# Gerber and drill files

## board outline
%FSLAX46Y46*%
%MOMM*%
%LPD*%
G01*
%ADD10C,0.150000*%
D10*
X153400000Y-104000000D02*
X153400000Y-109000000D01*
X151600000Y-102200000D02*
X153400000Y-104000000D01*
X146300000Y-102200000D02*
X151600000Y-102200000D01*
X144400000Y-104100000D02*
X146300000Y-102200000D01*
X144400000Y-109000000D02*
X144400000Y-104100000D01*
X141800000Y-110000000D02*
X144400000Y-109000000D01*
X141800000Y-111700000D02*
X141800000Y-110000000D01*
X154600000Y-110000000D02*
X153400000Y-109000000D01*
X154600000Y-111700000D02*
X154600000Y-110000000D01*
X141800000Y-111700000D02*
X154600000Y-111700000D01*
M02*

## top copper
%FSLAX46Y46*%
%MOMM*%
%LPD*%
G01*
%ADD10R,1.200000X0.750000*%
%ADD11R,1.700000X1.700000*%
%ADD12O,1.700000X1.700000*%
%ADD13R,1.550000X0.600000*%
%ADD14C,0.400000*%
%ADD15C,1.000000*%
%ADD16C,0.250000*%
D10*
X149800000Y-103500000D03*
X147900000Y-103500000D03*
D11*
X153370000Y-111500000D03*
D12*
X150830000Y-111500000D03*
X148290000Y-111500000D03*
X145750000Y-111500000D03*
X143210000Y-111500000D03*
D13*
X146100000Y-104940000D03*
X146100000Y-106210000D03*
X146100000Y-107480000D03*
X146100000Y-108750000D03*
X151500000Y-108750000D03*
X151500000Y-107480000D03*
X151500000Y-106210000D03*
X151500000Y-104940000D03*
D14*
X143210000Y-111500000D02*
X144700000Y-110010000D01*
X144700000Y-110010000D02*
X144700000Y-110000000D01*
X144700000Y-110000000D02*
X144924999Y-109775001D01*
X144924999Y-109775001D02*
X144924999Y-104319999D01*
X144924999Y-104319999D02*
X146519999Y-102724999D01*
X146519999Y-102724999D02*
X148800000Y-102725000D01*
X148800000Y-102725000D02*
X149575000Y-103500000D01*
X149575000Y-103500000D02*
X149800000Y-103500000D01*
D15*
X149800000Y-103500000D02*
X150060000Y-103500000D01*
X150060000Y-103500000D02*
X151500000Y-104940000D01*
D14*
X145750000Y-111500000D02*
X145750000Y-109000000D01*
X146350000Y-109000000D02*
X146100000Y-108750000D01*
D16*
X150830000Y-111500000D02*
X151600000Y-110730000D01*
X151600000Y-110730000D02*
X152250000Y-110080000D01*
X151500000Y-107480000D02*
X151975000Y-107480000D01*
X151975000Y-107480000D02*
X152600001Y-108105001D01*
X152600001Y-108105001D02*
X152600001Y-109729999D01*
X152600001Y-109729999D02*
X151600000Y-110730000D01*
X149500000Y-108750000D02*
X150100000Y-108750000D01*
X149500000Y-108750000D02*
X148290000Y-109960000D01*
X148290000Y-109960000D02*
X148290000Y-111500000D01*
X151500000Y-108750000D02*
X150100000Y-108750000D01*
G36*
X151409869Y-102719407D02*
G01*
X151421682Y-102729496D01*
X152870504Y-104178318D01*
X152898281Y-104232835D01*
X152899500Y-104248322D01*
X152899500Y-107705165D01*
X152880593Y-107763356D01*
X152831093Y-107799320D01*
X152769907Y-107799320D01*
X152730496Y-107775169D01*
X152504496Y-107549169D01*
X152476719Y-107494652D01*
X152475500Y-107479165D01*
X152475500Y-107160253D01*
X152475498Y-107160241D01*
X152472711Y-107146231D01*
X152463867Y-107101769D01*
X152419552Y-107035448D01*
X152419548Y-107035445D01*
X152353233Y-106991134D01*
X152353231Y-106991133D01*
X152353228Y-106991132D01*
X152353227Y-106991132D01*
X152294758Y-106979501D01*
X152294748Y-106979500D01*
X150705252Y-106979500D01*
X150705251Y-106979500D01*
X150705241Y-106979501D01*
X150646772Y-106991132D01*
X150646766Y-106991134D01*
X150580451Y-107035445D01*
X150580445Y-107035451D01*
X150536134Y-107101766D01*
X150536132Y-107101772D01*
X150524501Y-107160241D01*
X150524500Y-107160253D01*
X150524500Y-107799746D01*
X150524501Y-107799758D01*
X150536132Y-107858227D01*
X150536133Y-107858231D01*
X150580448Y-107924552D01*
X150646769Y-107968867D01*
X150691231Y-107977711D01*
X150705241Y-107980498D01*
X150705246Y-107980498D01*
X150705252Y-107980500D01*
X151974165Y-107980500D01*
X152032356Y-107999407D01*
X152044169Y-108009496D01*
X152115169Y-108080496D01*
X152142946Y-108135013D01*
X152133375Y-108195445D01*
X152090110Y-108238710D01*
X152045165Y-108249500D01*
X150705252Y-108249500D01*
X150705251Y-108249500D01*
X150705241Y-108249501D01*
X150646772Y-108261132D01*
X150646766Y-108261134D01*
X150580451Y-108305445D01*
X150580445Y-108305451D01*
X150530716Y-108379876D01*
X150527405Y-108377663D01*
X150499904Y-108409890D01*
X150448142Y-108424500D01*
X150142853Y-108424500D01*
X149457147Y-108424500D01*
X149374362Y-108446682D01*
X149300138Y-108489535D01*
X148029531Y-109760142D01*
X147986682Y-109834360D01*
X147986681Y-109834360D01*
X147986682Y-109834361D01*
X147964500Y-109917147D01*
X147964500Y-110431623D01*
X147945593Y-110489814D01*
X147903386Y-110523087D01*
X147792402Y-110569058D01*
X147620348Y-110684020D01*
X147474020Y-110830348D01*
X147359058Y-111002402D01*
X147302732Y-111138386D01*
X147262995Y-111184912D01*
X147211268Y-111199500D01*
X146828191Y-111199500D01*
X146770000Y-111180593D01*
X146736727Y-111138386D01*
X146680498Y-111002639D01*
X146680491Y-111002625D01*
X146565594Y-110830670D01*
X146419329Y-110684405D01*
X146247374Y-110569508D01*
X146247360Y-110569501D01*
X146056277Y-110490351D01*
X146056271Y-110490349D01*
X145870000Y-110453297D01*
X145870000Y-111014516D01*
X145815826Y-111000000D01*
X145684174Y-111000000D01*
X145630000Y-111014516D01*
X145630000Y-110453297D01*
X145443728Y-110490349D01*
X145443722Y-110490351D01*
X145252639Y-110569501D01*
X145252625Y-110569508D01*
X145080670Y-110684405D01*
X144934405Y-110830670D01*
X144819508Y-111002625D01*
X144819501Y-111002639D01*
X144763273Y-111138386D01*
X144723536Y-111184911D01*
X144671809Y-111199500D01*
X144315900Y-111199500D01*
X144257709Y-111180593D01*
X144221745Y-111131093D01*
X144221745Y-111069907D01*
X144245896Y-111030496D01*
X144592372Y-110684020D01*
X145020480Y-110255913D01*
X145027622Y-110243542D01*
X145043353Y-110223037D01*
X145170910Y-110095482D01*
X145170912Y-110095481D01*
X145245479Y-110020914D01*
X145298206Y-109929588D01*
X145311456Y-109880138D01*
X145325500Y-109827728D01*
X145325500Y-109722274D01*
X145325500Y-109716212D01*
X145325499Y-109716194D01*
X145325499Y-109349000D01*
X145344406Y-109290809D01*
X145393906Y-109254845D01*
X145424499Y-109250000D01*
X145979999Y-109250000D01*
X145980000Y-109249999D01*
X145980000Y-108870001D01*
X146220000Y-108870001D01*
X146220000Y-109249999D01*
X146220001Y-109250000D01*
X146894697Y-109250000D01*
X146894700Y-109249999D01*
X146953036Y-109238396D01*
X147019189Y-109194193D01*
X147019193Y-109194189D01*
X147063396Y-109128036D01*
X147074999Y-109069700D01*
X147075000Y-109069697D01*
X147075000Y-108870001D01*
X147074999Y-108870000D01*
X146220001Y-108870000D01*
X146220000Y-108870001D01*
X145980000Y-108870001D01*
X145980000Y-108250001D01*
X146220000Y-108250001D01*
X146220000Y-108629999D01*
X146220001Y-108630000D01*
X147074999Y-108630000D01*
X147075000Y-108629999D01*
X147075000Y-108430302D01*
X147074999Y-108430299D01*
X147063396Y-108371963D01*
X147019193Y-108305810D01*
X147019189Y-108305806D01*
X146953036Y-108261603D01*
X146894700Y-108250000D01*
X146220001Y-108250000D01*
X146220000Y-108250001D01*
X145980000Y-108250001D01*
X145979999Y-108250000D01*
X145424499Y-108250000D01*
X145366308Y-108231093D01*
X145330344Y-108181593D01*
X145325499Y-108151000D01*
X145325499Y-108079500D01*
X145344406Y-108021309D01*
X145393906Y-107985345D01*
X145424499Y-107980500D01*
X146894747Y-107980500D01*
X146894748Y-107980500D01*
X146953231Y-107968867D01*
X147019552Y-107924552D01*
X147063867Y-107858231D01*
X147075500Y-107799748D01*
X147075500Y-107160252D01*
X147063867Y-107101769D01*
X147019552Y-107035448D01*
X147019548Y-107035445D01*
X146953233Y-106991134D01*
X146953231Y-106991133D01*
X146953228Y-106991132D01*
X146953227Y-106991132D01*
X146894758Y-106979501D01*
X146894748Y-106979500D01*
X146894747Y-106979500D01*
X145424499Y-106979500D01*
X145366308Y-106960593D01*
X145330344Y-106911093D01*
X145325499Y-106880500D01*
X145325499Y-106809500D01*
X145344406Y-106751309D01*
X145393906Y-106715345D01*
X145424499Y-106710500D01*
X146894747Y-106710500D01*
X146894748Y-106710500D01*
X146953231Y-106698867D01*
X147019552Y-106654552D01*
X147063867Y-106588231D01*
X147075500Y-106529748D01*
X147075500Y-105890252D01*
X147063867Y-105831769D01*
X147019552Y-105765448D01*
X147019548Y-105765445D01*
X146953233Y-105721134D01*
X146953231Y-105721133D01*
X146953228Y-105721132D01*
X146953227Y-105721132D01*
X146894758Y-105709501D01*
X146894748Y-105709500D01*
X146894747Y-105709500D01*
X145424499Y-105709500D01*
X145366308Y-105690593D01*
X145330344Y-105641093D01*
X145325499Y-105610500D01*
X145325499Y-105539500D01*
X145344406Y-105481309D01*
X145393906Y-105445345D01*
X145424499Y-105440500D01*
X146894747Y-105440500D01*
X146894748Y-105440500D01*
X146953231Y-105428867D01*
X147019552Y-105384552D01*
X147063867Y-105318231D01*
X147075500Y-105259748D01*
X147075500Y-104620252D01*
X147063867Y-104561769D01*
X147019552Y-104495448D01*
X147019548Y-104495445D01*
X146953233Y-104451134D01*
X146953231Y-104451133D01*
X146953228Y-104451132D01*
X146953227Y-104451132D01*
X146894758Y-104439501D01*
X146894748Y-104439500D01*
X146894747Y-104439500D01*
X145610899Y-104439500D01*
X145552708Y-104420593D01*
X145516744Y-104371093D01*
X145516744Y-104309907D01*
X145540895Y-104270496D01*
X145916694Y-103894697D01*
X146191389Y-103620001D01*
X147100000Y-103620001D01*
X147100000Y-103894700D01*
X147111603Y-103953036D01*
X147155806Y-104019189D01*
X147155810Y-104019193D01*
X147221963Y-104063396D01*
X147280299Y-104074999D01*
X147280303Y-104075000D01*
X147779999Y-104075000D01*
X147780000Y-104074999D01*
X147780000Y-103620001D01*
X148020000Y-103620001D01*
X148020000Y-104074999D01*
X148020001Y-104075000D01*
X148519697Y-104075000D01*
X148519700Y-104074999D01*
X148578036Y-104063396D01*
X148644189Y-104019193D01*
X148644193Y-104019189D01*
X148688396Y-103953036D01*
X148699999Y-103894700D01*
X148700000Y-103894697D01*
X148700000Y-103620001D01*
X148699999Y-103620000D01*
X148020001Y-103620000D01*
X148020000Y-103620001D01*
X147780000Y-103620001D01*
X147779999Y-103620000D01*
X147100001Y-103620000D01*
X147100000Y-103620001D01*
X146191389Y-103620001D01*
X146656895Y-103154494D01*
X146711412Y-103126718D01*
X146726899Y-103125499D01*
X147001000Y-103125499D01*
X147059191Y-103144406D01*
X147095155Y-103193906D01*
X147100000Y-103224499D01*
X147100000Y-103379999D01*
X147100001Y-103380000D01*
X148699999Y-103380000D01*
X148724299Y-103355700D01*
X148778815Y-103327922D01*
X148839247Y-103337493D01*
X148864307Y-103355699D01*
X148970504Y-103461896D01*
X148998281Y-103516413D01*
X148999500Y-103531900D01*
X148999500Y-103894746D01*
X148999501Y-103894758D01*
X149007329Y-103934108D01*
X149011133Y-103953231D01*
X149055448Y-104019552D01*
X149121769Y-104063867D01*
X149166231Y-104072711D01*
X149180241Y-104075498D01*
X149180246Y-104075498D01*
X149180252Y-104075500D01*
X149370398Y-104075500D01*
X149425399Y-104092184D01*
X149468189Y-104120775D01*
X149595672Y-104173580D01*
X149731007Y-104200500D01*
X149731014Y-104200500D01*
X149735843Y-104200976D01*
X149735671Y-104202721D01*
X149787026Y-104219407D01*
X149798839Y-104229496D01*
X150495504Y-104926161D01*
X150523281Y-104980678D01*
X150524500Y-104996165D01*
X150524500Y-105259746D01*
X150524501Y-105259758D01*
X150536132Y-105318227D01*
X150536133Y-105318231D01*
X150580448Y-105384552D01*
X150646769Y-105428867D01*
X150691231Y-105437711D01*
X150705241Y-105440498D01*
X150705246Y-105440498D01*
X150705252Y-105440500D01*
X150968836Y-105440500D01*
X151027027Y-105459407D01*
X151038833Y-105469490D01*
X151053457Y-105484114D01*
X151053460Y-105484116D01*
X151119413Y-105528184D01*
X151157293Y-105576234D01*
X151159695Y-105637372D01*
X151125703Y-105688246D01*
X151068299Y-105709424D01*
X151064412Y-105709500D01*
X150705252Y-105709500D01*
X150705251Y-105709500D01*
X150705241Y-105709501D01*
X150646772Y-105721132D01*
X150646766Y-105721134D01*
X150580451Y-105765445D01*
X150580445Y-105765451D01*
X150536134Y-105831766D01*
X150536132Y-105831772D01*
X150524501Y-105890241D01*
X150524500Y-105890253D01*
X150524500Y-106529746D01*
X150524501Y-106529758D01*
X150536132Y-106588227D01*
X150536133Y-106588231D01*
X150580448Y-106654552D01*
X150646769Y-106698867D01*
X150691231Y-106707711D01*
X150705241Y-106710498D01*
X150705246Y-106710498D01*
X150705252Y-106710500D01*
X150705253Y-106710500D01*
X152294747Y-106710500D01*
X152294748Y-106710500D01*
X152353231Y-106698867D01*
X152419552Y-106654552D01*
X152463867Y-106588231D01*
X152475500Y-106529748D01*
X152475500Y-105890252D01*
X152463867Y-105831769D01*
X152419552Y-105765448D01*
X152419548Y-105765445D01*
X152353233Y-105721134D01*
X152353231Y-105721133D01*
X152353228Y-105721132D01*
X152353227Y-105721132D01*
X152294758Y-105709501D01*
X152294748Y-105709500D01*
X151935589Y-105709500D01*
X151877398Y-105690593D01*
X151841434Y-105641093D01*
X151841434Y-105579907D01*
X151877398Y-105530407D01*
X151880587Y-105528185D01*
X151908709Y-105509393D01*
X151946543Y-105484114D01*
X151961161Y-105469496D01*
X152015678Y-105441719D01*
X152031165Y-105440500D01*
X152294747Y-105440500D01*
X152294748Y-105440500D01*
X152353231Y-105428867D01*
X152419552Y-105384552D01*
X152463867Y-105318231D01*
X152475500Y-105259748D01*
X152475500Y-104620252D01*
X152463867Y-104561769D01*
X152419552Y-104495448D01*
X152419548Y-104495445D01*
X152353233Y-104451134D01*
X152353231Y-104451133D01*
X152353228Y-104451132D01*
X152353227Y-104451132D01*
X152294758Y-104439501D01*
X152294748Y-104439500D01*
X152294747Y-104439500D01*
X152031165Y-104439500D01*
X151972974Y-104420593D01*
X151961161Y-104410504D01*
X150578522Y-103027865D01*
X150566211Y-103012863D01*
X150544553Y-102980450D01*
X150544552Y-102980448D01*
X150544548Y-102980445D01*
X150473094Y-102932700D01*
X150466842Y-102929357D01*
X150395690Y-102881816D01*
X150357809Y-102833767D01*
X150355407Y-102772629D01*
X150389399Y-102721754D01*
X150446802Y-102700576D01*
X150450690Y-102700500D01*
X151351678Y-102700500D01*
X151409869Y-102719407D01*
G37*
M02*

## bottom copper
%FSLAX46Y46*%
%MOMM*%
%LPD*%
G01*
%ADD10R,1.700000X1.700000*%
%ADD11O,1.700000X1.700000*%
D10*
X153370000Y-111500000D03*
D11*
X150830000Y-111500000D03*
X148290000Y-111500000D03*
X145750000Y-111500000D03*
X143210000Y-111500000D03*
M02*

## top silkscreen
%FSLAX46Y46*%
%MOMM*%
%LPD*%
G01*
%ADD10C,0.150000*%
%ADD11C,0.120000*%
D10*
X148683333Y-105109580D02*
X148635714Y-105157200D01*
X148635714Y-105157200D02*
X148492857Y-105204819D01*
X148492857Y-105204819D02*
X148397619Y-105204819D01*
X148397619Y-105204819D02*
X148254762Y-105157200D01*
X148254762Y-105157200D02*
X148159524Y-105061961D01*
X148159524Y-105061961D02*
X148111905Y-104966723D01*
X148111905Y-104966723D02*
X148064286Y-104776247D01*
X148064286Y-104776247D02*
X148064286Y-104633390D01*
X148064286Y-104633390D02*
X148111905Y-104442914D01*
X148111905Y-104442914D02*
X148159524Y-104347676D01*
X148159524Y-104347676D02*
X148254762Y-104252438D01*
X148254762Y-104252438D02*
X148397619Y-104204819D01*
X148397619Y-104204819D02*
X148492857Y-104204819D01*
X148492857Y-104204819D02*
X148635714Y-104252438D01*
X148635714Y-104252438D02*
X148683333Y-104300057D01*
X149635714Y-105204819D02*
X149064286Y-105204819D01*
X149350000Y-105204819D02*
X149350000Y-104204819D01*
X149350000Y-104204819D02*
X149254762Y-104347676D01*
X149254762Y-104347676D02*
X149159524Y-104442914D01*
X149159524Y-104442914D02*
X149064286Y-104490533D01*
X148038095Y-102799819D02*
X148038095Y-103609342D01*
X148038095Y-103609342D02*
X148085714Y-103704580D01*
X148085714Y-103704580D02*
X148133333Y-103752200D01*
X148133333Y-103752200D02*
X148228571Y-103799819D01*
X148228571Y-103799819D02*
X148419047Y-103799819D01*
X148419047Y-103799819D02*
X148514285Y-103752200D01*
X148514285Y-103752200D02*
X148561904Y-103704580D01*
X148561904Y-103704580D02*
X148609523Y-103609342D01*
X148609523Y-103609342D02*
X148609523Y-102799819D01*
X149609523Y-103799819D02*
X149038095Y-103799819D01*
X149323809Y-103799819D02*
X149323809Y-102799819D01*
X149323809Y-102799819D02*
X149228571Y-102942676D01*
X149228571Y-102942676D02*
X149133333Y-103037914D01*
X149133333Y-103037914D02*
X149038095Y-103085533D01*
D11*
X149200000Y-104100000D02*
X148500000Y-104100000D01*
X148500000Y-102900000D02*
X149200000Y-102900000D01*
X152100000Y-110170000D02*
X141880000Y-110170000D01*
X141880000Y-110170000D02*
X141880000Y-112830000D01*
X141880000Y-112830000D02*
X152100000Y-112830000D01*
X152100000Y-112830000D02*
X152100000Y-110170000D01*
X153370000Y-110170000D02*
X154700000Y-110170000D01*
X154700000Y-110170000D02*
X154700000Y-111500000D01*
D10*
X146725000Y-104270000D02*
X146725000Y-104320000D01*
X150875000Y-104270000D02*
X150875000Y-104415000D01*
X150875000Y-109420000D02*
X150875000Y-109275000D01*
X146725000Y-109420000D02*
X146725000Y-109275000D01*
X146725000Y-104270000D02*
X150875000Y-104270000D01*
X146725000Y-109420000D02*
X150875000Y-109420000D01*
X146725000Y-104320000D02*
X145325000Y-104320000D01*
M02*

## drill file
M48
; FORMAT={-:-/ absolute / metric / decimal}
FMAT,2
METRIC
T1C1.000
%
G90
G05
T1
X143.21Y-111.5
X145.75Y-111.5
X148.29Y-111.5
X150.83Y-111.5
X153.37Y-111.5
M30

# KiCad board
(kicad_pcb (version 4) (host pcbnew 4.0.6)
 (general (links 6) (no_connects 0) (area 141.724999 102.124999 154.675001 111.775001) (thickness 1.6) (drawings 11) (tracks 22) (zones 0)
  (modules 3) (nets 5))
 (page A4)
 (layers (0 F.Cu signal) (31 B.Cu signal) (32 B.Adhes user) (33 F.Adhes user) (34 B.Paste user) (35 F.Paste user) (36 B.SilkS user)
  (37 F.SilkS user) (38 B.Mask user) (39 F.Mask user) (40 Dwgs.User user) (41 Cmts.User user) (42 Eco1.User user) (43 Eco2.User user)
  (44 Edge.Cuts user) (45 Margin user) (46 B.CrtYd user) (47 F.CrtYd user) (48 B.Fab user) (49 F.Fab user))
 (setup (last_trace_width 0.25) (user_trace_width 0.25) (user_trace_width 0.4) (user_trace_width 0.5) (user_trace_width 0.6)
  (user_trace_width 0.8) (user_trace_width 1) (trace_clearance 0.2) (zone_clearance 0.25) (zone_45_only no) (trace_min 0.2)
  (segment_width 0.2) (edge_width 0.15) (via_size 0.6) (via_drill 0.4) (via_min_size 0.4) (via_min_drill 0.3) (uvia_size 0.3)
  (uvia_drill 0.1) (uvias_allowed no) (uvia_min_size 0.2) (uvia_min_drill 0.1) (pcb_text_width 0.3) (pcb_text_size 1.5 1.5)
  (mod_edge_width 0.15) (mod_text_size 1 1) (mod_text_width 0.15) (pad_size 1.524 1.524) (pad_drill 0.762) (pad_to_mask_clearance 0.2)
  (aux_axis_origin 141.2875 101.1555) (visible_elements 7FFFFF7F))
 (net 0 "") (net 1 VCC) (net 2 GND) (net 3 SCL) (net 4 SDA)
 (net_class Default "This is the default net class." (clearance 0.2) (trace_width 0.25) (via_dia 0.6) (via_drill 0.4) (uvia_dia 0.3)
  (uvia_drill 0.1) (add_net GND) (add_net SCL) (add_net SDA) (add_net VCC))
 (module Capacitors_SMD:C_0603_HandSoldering (layer F.Cu) (at 148.85 103.5 180)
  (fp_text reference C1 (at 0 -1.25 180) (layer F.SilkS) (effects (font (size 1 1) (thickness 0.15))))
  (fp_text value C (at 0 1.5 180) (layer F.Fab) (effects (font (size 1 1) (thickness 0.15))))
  (fp_line (start -0.35 -0.6) (end 0.35 -0.6) (layer F.SilkS) (width 0.12))
  (fp_line (start 0.35 0.6) (end -0.35 0.6) (layer F.SilkS) (width 0.12))
  (pad 1 smd rect (at -0.95 0 180) (size 1.2 0.75) (layers F.Cu F.Paste F.Mask) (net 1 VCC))
  (pad 2 smd rect (at 0.95 0 180) (size 1.2 0.75) (layers F.Cu F.Paste F.Mask) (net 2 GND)))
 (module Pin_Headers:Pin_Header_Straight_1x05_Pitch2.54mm (layer F.Cu) (at 153.37 111.5 270)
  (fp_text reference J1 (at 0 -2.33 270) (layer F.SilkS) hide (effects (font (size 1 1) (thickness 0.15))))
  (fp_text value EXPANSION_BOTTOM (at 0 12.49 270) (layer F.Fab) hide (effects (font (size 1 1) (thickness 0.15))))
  (fp_line (start -1.33 1.27) (end -1.33 11.49) (layer F.SilkS) (width 0.12))
  (fp_line (start -1.33 11.49) (end 1.33 11.49) (layer F.SilkS) (width 0.12))
  (fp_line (start 1.33 11.49) (end 1.33 1.27) (layer F.SilkS) (width 0.12))
  (fp_line (start 1.33 1.27) (end -1.33 1.27) (layer F.SilkS) (width 0.12))
  (fp_line (start -1.33 0) (end -1.33 -1.33) (layer F.SilkS) (width 0.12))
  (fp_line (start -1.33 -1.33) (end 0 -1.33) (layer F.SilkS) (width 0.12))
  (pad 1 thru_hole rect (at 0 0 270) (size 1.7 1.7) (drill 1) (layers *.Cu *.Mask))
  (pad 2 thru_hole oval (at 0 2.54 270) (size 1.7 1.7) (drill 1) (layers *.Cu *.Mask) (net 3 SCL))
  (pad 3 thru_hole oval (at 0 5.08 270) (size 1.7 1.7) (drill 1) (layers *.Cu *.Mask) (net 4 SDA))
  (pad 4 thru_hole oval (at 0 7.62 270) (size 1.7 1.7) (drill 1) (layers *.Cu *.Mask) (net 2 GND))
  (pad 5 thru_hole oval (at 0 10.16 270) (size 1.7 1.7) (drill 1) (layers *.Cu *.Mask) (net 1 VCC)))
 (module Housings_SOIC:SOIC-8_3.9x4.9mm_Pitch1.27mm (layer F.Cu) (at 148.8 106.845)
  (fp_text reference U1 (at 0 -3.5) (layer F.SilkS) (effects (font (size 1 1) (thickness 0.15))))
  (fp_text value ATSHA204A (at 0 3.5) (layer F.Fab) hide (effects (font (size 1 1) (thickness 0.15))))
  (fp_line (start -2.075 -2.575) (end -2.075 -2.525) (layer F.SilkS) (width 0.15))
  (fp_line (start 2.075 -2.575) (end 2.075 -2.43) (layer F.SilkS) (width 0.15))
  (fp_line (start 2.075 2.575) (end 2.075 2.43) (layer F.SilkS) (width 0.15))
  (fp_line (start -2.075 2.575) (end -2.075 2.43) (layer F.SilkS) (width 0.15))
  (fp_line (start -2.075 -2.575) (end 2.075 -2.575) (layer F.SilkS) (width 0.15))
  (fp_line (start -2.075 2.575) (end 2.075 2.575) (layer F.SilkS) (width 0.15))
  (fp_line (start -2.075 -2.525) (end -3.475 -2.525) (layer F.SilkS) (width 0.15))
  (pad 1 smd rect (at -2.7 -1.905) (size 1.55 0.6) (layers F.Cu F.Paste F.Mask))
  (pad 2 smd rect (at -2.7 -0.635) (size 1.55 0.6) (layers F.Cu F.Paste F.Mask))
  (pad 3 smd rect (at -2.7 0.635) (size 1.55 0.6) (layers F.Cu F.Paste F.Mask))
  (pad 4 smd rect (at -2.7 1.905) (size 1.55 0.6) (layers F.Cu F.Paste F.Mask) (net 2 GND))
  (pad 5 smd rect (at 2.7 1.905) (size 1.55 0.6) (layers F.Cu F.Paste F.Mask) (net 4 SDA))
  (pad 6 smd rect (at 2.7 0.635) (size 1.55 0.6) (layers F.Cu F.Paste F.Mask) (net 3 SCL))
  (pad 7 smd rect (at 2.7 -0.635) (size 1.55 0.6) (layers F.Cu F.Paste F.Mask))
  (pad 8 smd rect (at 2.7 -1.905) (size 1.55 0.6) (layers F.Cu F.Paste F.Mask) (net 1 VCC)))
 (gr_line (start 153.4 104) (end 153.4 109) (layer Edge.Cuts) (width 0.15))
 (gr_line (start 151.6 102.2) (end 153.4 104) (layer Edge.Cuts) (width 0.15))
 (gr_line (start 146.3 102.2) (end 151.6 102.2) (layer Edge.Cuts) (width 0.15))
 (gr_line (start 144.4 104.1) (end 146.3 102.2) (layer Edge.Cuts) (width 0.15))
 (gr_line (start 144.4 109) (end 144.4 104.1) (layer Edge.Cuts) (width 0.15))
 (gr_line (start 141.8 110) (end 144.4 109) (layer Edge.Cuts) (width 0.15))
 (gr_line (start 141.8 111.7) (end 141.8 110) (layer Edge.Cuts) (width 0.15))
 (gr_line (start 154.6 110) (end 153.4 109) (layer Edge.Cuts) (width 0.15))
 (gr_line (start 154.6 111.7) (end 154.6 110) (layer Edge.Cuts) (width 0.15))
 (gr_line (start 141.8 111.7) (end 154.6 111.7) (layer Edge.Cuts) (width 0.15))
 (segment (start 143.21 111.5) (end 144.7 110.01) (width 0.4) (layer F.Cu) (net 1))
 (segment (start 144.7 110.01) (end 144.7 110) (width 0.4) (layer F.Cu) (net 1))
 (segment (start 144.7 110) (end 144.924999 109.775001) (width 0.4) (layer F.Cu) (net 1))
 (segment (start 144.924999 109.775001) (end 144.924999 104.319999) (width 0.4) (layer F.Cu) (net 1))
 (segment (start 144.924999 104.319999) (end 146.519999 102.724999) (width 0.4) (layer F.Cu) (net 1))
 (segment (start 146.519999 102.724999) (end 148.8 102.725) (width 0.4) (layer F.Cu) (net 1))
 (segment (start 148.8 102.725) (end 149.575 103.5) (width 0.4) (layer F.Cu) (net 1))
 (segment (start 149.575 103.5) (end 149.8 103.5) (width 0.4) (layer F.Cu) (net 1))
 (segment (start 149.8 103.5) (end 150.06 103.5) (width 1) (layer F.Cu) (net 1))
 (segment (start 150.06 103.5) (end 151.5 104.94) (width 1) (layer F.Cu) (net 1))
 (segment (start 145.75 111.5) (end 145.75 109) (width 0.4) (layer F.Cu) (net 2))
 (segment (start 146.35 109) (end 146.1 108.75) (width 0.4) (layer F.Cu) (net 2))
 (segment (start 150.83 111.5) (end 151.6 110.73) (width 0.25) (layer F.Cu) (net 3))
 (segment (start 151.6 110.73) (end 152.25 110.08) (width 0.25) (layer F.Cu) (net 3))
 (segment (start 151.5 107.48) (end 151.975 107.48) (width 0.25) (layer F.Cu) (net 3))
 (segment (start 151.975 107.48) (end 152.600001 108.105001) (width 0.25) (layer F.Cu) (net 3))
 (segment (start 152.600001 108.105001) (end 152.600001 109.729999) (width 0.25) (layer F.Cu) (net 3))
 (segment (start 152.600001 109.729999) (end 151.6 110.73) (width 0.25) (layer F.Cu) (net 3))
 (segment (start 149.5 108.75) (end 150.1 108.75) (width 0.25) (layer F.Cu) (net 4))
 (segment (start 149.5 108.75) (end 148.29 109.96) (width 0.25) (layer F.Cu) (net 4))
 (segment (start 148.29 109.96) (end 148.29 111.5) (width 0.25) (layer F.Cu) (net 4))
 (segment (start 151.5 108.75) (end 150.1 108.75) (width 0.25) (layer F.Cu) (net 4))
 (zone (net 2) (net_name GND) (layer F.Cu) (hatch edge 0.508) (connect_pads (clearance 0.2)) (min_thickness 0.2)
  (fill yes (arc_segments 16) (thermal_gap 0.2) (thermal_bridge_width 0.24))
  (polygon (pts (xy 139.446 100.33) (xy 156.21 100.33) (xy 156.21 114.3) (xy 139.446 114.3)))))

